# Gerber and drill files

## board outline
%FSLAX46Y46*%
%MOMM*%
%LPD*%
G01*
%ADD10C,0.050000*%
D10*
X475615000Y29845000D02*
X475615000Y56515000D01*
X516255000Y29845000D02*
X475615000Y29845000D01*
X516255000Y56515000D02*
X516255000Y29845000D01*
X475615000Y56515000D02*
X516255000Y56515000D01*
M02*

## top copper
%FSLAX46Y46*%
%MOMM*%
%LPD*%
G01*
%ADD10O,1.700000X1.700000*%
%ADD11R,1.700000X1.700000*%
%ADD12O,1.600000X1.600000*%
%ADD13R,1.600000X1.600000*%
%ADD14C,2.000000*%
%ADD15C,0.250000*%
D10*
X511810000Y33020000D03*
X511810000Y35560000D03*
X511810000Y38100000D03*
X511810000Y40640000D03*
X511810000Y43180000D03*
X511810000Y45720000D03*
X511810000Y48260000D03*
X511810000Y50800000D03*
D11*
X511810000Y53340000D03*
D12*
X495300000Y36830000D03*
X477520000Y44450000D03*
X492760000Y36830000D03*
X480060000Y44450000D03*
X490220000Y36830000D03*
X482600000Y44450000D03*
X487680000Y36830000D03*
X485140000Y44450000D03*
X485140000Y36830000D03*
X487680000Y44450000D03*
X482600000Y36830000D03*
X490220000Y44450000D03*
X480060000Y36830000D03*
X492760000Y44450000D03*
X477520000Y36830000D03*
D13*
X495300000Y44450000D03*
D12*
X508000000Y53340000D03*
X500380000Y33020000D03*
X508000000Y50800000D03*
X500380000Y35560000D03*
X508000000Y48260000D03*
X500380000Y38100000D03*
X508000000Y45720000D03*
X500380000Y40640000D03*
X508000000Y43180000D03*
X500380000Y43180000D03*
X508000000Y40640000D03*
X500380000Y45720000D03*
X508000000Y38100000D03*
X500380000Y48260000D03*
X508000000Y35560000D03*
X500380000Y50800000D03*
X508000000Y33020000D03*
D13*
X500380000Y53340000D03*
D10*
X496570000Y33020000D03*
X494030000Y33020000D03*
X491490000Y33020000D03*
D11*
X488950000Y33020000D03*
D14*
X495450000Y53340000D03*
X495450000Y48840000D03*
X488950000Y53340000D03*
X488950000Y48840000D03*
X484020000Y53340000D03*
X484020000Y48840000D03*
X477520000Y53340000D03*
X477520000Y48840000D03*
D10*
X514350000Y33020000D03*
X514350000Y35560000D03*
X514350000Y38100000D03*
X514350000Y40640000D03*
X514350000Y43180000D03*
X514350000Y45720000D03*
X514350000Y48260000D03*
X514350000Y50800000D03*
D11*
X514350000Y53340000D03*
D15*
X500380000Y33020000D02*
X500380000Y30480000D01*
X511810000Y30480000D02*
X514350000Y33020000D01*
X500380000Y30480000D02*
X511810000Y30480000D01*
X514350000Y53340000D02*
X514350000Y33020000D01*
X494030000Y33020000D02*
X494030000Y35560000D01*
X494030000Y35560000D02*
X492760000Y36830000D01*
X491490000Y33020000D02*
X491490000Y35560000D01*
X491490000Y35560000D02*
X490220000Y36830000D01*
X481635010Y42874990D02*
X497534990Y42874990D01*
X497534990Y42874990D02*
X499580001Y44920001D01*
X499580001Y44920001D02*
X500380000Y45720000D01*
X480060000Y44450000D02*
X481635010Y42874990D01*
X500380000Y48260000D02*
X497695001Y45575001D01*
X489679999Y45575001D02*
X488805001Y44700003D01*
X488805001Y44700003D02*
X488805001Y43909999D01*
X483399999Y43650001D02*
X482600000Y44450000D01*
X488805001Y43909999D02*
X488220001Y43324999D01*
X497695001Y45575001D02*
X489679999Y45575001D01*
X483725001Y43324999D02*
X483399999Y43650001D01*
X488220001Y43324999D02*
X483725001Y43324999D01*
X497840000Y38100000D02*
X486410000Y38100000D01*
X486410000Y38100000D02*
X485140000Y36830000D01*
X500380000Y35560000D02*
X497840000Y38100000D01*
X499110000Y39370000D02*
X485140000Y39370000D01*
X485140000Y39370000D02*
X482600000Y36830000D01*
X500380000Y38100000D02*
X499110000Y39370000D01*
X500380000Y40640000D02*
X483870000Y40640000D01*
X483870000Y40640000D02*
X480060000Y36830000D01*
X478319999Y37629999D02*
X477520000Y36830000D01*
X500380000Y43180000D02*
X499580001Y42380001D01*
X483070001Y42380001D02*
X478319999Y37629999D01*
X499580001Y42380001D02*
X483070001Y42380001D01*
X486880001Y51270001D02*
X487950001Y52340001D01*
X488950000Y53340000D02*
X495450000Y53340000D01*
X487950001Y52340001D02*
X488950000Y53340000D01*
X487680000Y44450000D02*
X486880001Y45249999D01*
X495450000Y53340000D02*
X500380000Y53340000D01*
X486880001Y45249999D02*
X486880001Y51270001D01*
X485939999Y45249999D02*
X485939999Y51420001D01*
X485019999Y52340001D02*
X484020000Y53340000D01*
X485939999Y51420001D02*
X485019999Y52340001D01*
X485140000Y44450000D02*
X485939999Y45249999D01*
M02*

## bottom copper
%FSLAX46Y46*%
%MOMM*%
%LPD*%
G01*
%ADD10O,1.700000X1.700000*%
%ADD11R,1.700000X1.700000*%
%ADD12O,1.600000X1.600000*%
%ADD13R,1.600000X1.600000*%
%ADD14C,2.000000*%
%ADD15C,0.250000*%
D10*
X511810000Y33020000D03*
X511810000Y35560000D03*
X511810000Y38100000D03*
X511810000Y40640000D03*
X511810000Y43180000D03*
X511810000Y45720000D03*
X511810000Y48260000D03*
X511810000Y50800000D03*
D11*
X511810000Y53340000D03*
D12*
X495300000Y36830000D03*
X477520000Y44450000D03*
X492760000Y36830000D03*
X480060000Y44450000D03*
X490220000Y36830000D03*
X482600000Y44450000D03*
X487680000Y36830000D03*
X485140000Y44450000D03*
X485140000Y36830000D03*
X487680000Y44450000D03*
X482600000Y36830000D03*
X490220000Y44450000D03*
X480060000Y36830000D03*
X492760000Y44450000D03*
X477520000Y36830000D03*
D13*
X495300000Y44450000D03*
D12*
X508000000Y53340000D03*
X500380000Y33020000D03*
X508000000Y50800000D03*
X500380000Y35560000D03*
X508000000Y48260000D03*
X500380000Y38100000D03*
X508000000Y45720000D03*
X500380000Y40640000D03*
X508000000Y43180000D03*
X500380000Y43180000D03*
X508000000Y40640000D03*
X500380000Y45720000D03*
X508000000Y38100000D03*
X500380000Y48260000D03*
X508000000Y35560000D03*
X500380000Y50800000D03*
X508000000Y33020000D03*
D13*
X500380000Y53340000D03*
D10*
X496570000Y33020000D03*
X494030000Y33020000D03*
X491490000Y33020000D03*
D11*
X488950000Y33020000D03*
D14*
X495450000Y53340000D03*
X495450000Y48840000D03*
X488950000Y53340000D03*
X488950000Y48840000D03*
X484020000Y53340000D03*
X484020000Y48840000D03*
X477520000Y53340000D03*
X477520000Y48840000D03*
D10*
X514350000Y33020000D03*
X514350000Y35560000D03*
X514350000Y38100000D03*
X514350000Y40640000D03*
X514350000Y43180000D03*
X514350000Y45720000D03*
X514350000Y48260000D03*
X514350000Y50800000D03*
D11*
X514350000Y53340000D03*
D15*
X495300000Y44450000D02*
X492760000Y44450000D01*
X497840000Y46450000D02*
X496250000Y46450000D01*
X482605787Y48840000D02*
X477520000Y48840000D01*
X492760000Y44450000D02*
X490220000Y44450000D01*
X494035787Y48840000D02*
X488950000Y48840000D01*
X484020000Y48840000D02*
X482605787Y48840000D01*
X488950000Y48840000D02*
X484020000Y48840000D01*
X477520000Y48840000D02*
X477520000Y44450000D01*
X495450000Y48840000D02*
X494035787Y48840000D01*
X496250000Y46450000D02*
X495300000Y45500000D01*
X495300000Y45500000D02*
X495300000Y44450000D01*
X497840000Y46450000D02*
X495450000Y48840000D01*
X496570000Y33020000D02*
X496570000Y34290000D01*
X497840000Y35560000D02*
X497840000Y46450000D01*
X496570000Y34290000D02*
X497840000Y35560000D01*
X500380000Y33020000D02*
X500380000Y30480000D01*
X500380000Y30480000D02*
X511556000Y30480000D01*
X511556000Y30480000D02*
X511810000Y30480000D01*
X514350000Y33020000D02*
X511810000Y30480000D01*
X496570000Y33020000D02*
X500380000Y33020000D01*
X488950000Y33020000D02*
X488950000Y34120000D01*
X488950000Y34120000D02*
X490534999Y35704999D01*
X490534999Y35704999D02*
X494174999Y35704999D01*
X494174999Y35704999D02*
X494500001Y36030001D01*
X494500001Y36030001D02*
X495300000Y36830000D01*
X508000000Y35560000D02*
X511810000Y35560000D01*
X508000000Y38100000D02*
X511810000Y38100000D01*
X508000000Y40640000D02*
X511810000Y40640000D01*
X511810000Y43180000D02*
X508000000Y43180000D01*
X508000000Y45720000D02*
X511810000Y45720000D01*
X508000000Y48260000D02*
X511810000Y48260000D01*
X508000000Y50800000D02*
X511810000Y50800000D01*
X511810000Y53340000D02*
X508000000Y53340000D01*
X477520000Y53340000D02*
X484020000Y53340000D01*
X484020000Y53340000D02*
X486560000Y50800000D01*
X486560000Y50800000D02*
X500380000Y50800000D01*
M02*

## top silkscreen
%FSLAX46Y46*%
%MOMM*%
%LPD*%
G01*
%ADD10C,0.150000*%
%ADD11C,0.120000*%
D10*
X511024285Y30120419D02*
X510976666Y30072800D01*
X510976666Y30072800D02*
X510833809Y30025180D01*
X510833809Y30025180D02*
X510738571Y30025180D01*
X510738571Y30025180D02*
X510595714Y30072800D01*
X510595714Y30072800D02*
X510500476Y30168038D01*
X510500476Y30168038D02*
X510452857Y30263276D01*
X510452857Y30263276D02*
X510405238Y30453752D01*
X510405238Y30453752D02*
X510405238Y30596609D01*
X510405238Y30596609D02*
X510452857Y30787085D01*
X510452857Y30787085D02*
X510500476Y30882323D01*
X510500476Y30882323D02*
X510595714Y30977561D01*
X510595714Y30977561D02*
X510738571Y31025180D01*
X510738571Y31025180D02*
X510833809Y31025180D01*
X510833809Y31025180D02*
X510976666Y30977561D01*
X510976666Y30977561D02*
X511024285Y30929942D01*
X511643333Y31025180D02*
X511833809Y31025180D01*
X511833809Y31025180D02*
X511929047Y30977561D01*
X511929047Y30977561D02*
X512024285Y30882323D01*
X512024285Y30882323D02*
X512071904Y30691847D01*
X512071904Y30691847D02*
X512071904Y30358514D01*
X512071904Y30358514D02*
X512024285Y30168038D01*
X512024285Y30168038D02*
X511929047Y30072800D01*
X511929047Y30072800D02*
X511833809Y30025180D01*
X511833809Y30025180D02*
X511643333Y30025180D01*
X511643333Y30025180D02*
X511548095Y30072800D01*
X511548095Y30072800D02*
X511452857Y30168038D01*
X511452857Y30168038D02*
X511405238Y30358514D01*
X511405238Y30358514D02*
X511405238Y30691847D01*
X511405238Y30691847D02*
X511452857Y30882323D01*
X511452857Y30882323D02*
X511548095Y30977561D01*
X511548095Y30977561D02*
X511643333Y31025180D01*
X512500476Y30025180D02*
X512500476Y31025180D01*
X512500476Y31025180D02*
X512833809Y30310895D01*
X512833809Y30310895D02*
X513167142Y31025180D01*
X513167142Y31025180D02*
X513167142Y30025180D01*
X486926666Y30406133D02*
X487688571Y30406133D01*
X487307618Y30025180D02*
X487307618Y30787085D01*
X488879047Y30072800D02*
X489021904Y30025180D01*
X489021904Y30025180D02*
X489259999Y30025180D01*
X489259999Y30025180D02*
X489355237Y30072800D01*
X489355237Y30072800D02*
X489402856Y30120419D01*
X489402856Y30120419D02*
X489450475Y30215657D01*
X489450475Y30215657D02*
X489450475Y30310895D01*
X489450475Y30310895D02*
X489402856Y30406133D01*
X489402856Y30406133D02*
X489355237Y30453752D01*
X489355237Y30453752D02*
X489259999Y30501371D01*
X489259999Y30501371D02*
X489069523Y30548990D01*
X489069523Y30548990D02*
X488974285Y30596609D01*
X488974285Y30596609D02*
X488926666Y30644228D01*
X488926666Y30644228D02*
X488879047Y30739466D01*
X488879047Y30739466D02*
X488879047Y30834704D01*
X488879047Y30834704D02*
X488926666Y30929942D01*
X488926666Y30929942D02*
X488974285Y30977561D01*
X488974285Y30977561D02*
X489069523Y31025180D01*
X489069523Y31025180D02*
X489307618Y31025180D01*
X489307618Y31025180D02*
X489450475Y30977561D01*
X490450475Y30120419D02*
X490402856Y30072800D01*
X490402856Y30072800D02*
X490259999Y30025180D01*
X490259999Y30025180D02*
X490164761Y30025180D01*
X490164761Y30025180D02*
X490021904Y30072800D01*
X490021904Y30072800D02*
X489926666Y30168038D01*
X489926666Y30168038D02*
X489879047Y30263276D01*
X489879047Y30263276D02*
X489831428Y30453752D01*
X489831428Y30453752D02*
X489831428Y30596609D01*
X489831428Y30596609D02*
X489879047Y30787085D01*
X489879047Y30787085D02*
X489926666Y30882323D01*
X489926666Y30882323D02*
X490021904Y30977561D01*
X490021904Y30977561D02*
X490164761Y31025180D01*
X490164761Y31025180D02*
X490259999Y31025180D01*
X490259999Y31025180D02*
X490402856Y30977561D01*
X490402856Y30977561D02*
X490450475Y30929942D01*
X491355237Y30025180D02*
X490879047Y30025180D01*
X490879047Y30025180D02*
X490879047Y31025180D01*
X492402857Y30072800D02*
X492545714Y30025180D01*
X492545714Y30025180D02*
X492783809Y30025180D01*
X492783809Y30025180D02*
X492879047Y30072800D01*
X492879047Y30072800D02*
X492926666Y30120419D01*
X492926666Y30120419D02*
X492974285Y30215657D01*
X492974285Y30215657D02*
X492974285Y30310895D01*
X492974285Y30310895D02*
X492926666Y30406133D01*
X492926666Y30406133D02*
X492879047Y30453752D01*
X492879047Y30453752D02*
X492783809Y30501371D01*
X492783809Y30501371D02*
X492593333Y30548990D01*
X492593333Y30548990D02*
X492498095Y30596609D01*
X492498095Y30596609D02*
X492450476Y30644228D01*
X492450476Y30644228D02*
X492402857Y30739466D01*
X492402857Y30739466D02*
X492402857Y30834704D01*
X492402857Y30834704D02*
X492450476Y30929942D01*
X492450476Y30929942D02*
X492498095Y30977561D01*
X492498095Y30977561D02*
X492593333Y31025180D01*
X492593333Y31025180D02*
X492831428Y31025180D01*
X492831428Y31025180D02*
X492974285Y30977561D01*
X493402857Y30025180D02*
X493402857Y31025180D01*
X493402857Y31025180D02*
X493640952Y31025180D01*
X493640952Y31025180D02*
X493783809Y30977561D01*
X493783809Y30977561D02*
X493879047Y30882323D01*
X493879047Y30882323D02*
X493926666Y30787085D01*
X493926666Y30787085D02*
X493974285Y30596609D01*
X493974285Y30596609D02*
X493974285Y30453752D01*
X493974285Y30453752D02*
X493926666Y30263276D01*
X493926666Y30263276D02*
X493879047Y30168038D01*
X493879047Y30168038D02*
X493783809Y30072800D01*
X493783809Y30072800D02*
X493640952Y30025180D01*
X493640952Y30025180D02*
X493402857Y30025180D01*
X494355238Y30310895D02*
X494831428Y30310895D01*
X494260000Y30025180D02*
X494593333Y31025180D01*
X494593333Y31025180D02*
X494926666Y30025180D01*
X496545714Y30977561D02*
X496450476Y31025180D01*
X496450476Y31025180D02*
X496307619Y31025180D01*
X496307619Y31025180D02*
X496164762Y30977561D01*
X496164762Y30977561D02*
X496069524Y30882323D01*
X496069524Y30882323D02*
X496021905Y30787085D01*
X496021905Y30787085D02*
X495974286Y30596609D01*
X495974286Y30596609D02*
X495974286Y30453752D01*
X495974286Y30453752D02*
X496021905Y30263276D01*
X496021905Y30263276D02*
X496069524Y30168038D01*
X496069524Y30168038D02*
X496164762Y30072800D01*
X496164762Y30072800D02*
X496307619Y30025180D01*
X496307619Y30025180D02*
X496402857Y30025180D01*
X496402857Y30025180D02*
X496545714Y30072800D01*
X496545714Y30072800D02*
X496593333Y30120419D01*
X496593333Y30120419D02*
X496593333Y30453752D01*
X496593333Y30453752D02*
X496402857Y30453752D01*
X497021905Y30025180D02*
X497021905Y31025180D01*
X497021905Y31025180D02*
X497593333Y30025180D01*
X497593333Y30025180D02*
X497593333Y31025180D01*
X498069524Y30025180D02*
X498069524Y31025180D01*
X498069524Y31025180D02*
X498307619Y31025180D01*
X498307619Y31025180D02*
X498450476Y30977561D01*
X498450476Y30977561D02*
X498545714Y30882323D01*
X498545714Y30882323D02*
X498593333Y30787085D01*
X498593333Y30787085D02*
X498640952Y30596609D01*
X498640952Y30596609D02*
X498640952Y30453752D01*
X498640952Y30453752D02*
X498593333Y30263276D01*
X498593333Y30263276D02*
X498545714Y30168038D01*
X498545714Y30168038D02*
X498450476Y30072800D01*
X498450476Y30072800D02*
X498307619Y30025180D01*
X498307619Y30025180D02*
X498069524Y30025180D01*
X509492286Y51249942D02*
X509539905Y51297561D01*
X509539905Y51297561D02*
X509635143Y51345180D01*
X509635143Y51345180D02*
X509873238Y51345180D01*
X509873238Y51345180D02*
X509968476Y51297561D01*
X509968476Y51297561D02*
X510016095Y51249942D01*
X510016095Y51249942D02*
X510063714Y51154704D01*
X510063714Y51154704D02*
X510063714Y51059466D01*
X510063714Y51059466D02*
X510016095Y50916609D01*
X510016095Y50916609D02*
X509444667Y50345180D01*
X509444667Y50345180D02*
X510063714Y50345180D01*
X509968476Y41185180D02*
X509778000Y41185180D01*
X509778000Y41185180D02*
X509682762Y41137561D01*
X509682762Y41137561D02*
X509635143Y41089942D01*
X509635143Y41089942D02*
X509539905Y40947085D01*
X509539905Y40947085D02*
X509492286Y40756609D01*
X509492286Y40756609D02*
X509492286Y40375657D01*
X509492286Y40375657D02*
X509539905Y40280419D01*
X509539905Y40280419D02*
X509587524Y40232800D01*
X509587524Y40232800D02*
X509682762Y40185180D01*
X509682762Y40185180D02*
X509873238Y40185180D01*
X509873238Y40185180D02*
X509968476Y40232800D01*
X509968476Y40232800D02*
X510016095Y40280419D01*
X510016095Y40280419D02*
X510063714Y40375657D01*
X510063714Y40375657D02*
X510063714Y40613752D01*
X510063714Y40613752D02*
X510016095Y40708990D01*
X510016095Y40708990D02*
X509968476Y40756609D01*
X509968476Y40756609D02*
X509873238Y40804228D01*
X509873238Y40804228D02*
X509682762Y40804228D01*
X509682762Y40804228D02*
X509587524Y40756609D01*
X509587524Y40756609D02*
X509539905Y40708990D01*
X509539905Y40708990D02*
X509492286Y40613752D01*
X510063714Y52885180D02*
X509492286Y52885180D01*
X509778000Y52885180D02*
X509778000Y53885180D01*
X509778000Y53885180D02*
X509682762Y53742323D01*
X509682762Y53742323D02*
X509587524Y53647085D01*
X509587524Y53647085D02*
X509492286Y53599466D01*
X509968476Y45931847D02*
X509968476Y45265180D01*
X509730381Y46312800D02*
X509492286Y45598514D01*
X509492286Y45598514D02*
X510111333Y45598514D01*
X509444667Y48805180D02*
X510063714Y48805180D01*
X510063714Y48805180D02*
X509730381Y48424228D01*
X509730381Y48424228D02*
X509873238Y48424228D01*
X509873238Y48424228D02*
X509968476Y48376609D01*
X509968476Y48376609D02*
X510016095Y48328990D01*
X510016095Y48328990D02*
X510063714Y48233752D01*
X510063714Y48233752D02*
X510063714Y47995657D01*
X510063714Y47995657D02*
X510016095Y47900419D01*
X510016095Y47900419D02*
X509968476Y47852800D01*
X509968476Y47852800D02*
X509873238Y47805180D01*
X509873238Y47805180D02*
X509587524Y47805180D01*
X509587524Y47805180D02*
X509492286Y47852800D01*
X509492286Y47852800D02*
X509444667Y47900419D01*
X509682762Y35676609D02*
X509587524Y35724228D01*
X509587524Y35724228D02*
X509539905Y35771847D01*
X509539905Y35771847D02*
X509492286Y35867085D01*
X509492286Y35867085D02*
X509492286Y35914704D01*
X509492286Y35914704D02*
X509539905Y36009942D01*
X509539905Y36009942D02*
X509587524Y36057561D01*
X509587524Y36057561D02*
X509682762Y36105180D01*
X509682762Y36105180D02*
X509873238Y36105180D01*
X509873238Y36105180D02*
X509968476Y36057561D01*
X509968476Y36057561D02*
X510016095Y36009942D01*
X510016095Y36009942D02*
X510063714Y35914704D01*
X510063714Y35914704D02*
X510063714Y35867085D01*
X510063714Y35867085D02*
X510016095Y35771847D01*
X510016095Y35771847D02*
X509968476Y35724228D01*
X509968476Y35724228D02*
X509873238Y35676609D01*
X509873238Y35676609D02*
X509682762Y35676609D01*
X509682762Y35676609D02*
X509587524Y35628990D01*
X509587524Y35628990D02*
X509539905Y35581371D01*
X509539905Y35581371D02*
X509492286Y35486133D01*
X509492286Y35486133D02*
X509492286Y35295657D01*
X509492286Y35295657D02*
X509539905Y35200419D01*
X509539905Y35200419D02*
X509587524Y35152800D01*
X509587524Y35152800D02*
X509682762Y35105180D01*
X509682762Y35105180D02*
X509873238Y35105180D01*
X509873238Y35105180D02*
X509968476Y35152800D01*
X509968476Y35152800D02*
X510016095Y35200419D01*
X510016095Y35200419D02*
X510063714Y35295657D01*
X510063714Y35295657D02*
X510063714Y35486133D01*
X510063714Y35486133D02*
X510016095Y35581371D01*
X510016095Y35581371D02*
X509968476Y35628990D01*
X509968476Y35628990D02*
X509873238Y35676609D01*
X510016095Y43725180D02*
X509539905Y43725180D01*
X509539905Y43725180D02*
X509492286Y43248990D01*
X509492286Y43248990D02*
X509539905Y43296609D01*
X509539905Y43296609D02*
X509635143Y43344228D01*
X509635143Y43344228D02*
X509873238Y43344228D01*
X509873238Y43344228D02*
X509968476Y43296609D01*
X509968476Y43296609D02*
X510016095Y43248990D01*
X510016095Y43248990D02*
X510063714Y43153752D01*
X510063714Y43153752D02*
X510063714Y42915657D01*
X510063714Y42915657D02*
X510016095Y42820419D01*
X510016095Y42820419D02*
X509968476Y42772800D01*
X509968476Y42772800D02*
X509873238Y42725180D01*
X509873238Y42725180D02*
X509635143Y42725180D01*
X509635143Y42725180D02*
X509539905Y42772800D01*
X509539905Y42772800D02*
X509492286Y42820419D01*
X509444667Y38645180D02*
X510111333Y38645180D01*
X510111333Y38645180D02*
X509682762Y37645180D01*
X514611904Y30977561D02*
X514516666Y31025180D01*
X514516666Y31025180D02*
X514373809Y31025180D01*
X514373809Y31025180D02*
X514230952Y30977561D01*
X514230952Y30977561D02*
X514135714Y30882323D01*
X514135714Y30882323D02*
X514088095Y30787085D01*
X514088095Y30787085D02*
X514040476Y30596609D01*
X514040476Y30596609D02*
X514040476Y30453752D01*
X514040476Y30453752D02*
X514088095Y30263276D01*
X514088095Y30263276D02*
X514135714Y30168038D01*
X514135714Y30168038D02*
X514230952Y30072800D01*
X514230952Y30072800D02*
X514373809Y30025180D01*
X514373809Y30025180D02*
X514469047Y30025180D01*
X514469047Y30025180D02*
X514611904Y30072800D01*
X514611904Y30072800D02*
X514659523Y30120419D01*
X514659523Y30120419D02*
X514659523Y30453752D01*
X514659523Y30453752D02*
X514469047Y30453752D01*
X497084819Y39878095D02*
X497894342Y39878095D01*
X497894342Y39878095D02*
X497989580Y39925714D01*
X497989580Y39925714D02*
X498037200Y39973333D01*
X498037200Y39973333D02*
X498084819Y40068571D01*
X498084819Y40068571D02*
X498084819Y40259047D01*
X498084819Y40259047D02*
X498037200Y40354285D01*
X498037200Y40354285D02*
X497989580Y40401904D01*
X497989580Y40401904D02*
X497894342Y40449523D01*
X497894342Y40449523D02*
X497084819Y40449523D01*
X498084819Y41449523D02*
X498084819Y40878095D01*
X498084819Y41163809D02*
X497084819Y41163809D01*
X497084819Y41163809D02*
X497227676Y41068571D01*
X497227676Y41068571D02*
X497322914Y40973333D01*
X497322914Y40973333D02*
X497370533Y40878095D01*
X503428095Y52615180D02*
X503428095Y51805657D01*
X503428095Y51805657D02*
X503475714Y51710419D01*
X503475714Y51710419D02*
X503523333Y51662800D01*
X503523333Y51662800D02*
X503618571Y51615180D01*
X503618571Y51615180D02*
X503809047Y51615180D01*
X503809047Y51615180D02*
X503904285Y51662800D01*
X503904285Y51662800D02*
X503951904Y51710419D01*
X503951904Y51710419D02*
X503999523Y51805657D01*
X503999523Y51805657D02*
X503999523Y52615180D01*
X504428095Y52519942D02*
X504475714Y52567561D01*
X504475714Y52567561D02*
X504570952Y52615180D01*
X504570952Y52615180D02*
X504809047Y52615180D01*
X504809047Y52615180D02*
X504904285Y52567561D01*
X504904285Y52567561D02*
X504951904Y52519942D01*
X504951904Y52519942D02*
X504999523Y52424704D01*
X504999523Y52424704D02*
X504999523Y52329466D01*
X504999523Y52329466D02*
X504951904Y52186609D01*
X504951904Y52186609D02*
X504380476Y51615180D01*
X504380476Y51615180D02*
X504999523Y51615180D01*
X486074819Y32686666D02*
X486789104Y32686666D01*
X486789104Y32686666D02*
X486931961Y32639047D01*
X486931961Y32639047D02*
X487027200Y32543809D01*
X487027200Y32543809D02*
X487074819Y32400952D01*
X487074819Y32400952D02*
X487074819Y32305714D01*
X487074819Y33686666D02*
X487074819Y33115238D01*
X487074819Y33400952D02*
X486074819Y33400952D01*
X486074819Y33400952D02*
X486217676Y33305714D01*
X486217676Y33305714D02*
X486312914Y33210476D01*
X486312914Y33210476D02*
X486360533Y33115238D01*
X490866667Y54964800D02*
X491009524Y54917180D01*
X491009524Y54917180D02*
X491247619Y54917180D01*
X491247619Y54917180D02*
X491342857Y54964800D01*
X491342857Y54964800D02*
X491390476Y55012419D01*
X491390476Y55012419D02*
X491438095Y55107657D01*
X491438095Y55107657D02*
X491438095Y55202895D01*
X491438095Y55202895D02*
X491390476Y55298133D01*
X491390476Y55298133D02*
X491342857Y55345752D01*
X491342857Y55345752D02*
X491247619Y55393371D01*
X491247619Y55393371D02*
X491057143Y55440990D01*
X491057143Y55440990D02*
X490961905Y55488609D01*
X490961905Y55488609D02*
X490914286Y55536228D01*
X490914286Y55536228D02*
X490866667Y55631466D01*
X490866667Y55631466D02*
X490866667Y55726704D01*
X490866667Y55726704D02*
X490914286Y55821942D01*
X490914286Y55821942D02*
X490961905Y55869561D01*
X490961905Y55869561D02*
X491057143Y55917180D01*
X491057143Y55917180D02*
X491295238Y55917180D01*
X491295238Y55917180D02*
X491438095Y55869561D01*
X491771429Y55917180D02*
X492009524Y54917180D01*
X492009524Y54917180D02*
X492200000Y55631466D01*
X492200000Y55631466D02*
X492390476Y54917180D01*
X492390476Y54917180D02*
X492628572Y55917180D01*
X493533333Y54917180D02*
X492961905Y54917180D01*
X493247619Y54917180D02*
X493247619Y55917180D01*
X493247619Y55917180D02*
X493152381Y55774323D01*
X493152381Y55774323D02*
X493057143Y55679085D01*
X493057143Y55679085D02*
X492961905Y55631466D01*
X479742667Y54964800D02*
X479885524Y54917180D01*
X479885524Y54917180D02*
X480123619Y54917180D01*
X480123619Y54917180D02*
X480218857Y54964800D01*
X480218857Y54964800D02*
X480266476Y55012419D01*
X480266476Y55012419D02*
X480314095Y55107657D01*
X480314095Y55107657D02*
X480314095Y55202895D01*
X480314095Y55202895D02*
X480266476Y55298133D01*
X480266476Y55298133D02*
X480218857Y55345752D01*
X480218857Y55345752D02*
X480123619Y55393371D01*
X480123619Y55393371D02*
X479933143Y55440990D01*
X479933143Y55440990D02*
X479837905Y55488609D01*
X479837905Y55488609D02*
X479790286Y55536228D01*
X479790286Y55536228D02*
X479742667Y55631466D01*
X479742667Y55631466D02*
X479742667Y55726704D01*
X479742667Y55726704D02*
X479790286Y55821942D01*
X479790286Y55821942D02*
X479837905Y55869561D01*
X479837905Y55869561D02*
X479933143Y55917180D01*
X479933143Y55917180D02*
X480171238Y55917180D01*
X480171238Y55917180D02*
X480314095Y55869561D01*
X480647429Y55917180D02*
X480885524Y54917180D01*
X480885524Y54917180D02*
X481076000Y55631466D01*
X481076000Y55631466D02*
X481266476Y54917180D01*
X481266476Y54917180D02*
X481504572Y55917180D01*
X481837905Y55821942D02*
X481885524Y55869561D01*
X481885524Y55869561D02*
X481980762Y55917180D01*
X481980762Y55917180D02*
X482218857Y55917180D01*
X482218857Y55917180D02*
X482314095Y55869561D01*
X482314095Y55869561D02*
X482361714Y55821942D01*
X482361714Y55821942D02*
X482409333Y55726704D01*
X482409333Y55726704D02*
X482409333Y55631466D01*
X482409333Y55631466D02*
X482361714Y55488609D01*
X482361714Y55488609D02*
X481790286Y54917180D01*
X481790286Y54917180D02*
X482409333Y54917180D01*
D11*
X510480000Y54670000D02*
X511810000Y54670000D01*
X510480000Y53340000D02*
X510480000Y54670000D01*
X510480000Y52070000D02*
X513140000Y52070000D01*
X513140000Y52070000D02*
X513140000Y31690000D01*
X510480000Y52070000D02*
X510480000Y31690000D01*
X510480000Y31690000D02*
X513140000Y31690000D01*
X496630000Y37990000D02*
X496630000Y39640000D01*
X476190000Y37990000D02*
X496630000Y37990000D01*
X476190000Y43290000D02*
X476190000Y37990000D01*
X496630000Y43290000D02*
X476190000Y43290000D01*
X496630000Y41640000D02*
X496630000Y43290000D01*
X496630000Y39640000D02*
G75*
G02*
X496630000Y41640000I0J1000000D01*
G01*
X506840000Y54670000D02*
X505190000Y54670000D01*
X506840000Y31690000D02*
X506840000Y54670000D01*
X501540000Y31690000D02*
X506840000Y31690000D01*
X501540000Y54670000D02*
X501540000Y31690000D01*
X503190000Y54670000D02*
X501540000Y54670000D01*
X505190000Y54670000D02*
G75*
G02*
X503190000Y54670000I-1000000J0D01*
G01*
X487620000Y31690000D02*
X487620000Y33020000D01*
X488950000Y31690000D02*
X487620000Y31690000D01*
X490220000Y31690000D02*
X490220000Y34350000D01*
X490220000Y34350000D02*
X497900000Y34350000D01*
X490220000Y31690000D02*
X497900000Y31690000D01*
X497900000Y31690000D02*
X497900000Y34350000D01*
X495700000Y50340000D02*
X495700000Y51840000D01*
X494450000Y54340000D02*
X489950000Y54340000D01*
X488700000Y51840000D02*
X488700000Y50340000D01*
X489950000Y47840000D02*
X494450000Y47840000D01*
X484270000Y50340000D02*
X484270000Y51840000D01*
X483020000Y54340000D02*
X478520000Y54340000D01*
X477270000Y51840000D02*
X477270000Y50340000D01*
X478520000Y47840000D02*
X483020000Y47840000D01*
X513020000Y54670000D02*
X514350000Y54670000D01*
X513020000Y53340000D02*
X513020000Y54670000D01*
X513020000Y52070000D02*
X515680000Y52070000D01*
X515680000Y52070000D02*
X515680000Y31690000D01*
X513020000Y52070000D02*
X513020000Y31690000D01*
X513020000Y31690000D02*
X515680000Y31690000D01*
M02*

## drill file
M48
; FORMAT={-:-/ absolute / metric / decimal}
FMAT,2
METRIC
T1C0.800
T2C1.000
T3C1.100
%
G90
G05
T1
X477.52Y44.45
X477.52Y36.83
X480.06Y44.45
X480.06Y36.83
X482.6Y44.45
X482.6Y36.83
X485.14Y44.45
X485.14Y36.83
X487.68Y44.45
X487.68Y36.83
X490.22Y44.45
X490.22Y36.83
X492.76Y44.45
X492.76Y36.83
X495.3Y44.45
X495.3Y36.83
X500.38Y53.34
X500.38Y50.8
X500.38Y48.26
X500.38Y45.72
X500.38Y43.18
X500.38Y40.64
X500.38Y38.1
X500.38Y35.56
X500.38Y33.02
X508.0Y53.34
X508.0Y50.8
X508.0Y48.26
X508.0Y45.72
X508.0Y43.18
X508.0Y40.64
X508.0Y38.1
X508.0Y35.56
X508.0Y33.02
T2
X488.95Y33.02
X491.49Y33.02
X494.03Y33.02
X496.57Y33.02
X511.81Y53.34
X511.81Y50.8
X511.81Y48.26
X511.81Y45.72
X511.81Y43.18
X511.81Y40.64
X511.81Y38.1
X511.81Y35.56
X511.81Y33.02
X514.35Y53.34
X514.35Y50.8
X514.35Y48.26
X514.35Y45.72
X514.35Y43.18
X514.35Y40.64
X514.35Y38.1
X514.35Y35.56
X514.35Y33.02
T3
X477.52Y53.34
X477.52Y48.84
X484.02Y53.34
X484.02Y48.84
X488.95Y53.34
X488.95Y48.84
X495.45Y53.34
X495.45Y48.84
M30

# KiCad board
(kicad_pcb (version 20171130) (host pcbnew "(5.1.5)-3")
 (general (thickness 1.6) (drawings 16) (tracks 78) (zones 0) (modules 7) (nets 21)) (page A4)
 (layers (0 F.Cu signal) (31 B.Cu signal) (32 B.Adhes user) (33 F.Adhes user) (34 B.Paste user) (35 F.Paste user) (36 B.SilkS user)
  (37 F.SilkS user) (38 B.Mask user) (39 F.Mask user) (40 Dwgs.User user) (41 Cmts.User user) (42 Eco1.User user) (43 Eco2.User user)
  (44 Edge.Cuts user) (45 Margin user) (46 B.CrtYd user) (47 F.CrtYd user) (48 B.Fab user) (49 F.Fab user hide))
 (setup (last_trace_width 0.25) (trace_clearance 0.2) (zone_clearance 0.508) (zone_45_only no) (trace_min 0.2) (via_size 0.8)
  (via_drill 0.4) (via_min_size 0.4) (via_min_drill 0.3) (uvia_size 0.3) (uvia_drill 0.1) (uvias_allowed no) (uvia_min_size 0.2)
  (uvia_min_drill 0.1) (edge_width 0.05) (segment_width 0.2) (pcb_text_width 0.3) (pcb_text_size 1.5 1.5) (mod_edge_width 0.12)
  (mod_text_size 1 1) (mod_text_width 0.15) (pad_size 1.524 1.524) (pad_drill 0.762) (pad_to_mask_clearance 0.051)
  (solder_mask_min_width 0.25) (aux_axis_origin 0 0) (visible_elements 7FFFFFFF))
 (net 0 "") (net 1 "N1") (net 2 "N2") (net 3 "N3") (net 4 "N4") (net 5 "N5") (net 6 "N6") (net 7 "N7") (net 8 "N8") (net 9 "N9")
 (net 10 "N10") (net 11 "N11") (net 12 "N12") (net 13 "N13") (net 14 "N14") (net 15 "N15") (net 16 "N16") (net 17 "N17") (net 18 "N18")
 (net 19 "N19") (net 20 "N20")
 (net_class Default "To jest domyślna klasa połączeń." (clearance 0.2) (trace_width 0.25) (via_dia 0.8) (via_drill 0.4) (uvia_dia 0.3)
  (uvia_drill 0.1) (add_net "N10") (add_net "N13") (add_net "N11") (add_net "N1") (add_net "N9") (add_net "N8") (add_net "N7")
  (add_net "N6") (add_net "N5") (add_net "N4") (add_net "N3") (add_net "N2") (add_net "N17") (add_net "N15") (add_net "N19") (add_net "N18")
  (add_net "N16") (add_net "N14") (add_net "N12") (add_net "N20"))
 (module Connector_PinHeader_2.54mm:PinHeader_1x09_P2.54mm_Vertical (layer F.Cu) (at 511.81 -53.34)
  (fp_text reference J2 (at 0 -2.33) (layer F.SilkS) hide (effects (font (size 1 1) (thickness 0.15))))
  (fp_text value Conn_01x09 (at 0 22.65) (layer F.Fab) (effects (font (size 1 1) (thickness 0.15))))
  (fp_line (start -1.33 -1.33) (end 0 -1.33) (layer F.SilkS) (width 0.12))
  (fp_line (start -1.33 0) (end -1.33 -1.33) (layer F.SilkS) (width 0.12))
  (fp_line (start -1.33 1.27) (end 1.33 1.27) (layer F.SilkS) (width 0.12))
  (fp_line (start 1.33 1.27) (end 1.33 21.65) (layer F.SilkS) (width 0.12))
  (fp_line (start -1.33 1.27) (end -1.33 21.65) (layer F.SilkS) (width 0.12))
  (fp_line (start -1.33 21.65) (end 1.33 21.65) (layer F.SilkS) (width 0.12))
  (pad 9 thru_hole oval (at 0 20.32) (size 1.7 1.7) (drill 1) (layers *.Cu *.Mask) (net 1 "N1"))
  (pad 8 thru_hole oval (at 0 17.78) (size 1.7 1.7) (drill 1) (layers *.Cu *.Mask) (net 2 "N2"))
  (pad 7 thru_hole oval (at 0 15.24) (size 1.7 1.7) (drill 1) (layers *.Cu *.Mask) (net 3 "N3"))
  (pad 6 thru_hole oval (at 0 12.7) (size 1.7 1.7) (drill 1) (layers *.Cu *.Mask) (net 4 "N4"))
  (pad 5 thru_hole oval (at 0 10.16) (size 1.7 1.7) (drill 1) (layers *.Cu *.Mask) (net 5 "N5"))
  (pad 4 thru_hole oval (at 0 7.62) (size 1.7 1.7) (drill 1) (layers *.Cu *.Mask) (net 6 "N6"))
  (pad 3 thru_hole oval (at 0 5.08) (size 1.7 1.7) (drill 1) (layers *.Cu *.Mask) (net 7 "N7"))
  (pad 2 thru_hole oval (at 0 2.54) (size 1.7 1.7) (drill 1) (layers *.Cu *.Mask) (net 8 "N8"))
  (pad 1 thru_hole rect (at 0 0) (size 1.7 1.7) (drill 1) (layers *.Cu *.Mask) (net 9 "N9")))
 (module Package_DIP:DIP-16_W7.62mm (layer F.Cu) (at 495.3 -44.45 270)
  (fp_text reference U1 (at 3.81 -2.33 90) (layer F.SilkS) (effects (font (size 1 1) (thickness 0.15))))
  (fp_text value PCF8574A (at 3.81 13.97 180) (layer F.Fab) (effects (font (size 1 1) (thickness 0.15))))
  (fp_line (start 6.46 -1.33) (end 4.81 -1.33) (layer F.SilkS) (width 0.12))
  (fp_line (start 6.46 19.11) (end 6.46 -1.33) (layer F.SilkS) (width 0.12))
  (fp_line (start 1.16 19.11) (end 6.46 19.11) (layer F.SilkS) (width 0.12))
  (fp_line (start 1.16 -1.33) (end 1.16 19.11) (layer F.SilkS) (width 0.12))
  (fp_line (start 2.81 -1.33) (end 1.16 -1.33) (layer F.SilkS) (width 0.12))
  (fp_arc (start 3.81 -1.33) (end 2.81 -1.33) (angle -180) (layer F.SilkS) (width 0.12))
  (pad 16 thru_hole oval (at 7.62 0 270) (size 1.6 1.6) (drill 0.8) (layers *.Cu *.Mask) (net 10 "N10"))
  (pad 8 thru_hole oval (at 0 17.78 270) (size 1.6 1.6) (drill 0.8) (layers *.Cu *.Mask) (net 1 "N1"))
  (pad 15 thru_hole oval (at 7.62 2.54 270) (size 1.6 1.6) (drill 0.8) (layers *.Cu *.Mask) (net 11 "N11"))
  (pad 7 thru_hole oval (at 0 15.24 270) (size 1.6 1.6) (drill 0.8) (layers *.Cu *.Mask) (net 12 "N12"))
  (pad 14 thru_hole oval (at 7.62 5.08 270) (size 1.6 1.6) (drill 0.8) (layers *.Cu *.Mask) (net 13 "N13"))
  (pad 6 thru_hole oval (at 0 12.7 270) (size 1.6 1.6) (drill 0.8) (layers *.Cu *.Mask) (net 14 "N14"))
  (pad 13 thru_hole oval (at 7.62 7.62 270) (size 1.6 1.6) (drill 0.8) (layers *.Cu *.Mask))
  (pad 5 thru_hole oval (at 0 10.16 270) (size 1.6 1.6) (drill 0.8) (layers *.Cu *.Mask) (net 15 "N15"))
  (pad 12 thru_hole oval (at 7.62 10.16 270) (size 1.6 1.6) (drill 0.8) (layers *.Cu *.Mask) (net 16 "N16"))
  (pad 4 thru_hole oval (at 0 7.62 270) (size 1.6 1.6) (drill 0.8) (layers *.Cu *.Mask) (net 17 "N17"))
  (pad 11 thru_hole oval (at 7.62 12.7 270) (size 1.6 1.6) (drill 0.8) (layers *.Cu *.Mask) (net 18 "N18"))
  (pad 3 thru_hole oval (at 0 5.08 270) (size 1.6 1.6) (drill 0.8) (layers *.Cu *.Mask) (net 1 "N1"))
  (pad 10 thru_hole oval (at 7.62 15.24 270) (size 1.6 1.6) (drill 0.8) (layers *.Cu *.Mask) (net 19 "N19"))
  (pad 2 thru_hole oval (at 0 2.54 270) (size 1.6 1.6) (drill 0.8) (layers *.Cu *.Mask) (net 1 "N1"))
  (pad 9 thru_hole oval (at 7.62 17.78 270) (size 1.6 1.6) (drill 0.8) (layers *.Cu *.Mask) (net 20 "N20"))
  (pad 1 thru_hole rect (at 0 0 270) (size 1.6 1.6) (drill 0.8) (layers *.Cu *.Mask) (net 1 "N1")))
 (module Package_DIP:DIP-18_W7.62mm (layer F.Cu) (at 500.38 -53.34)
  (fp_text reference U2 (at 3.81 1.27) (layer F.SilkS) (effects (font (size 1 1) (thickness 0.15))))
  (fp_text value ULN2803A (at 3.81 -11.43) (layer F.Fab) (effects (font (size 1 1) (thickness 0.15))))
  (fp_line (start 6.46 -1.33) (end 4.81 -1.33) (layer F.SilkS) (width 0.12))
  (fp_line (start 6.46 21.65) (end 6.46 -1.33) (layer F.SilkS) (width 0.12))
  (fp_line (start 1.16 21.65) (end 6.46 21.65) (layer F.SilkS) (width 0.12))
  (fp_line (start 1.16 -1.33) (end 1.16 21.65) (layer F.SilkS) (width 0.12))
  (fp_line (start 2.81 -1.33) (end 1.16 -1.33) (layer F.SilkS) (width 0.12))
  (fp_arc (start 3.81 -1.33) (end 2.81 -1.33) (angle -180) (layer F.SilkS) (width 0.12))
  (pad 18 thru_hole oval (at 7.62 0) (size 1.6 1.6) (drill 0.8) (layers *.Cu *.Mask) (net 9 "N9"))
  (pad 9 thru_hole oval (at 0 20.32) (size 1.6 1.6) (drill 0.8) (layers *.Cu *.Mask) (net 1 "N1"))
  (pad 17 thru_hole oval (at 7.62 2.54) (size 1.6 1.6) (drill 0.8) (layers *.Cu *.Mask) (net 8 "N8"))
  (pad 8 thru_hole oval (at 0 17.78) (size 1.6 1.6) (drill 0.8) (layers *.Cu *.Mask) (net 16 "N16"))
  (pad 16 thru_hole oval (at 7.62 5.08) (size 1.6 1.6) (drill 0.8) (layers *.Cu *.Mask) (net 7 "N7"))
  (pad 7 thru_hole oval (at 0 15.24) (size 1.6 1.6) (drill 0.8) (layers *.Cu *.Mask) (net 18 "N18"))
  (pad 15 thru_hole oval (at 7.62 7.62) (size 1.6 1.6) (drill 0.8) (layers *.Cu *.Mask) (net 6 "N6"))
  (pad 6 thru_hole oval (at 0 12.7) (size 1.6 1.6) (drill 0.8) (layers *.Cu *.Mask) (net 19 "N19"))
  (pad 14 thru_hole oval (at 7.62 10.16) (size 1.6 1.6) (drill 0.8) (layers *.Cu *.Mask) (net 5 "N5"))
  (pad 5 thru_hole oval (at 0 10.16) (size 1.6 1.6) (drill 0.8) (layers *.Cu *.Mask) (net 20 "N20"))
  (pad 13 thru_hole oval (at 7.62 12.7) (size 1.6 1.6) (drill 0.8) (layers *.Cu *.Mask) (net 4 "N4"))
  (pad 4 thru_hole oval (at 0 7.62) (size 1.6 1.6) (drill 0.8) (layers *.Cu *.Mask) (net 12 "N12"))
  (pad 12 thru_hole oval (at 7.62 15.24) (size 1.6 1.6) (drill 0.8) (layers *.Cu *.Mask) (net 3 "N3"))
  (pad 3 thru_hole oval (at 0 5.08) (size 1.6 1.6) (drill 0.8) (layers *.Cu *.Mask) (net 14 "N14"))
  (pad 11 thru_hole oval (at 7.62 17.78) (size 1.6 1.6) (drill 0.8) (layers *.Cu *.Mask) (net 2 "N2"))
  (pad 2 thru_hole oval (at 0 2.54) (size 1.6 1.6) (drill 0.8) (layers *.Cu *.Mask) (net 15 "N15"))
  (pad 10 thru_hole oval (at 7.62 20.32) (size 1.6 1.6) (drill 0.8) (layers *.Cu *.Mask))
  (pad 1 thru_hole rect (at 0 0) (size 1.6 1.6) (drill 0.8) (layers *.Cu *.Mask) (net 17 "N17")))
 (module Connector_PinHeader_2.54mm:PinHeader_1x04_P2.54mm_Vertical (layer F.Cu) (at 488.95 -33.02 90)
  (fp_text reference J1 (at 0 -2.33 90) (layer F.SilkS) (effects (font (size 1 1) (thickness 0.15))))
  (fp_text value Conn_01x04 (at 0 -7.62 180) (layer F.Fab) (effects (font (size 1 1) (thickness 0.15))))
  (fp_line (start -1.33 -1.33) (end 0 -1.33) (layer F.SilkS) (width 0.12))
  (fp_line (start -1.33 0) (end -1.33 -1.33) (layer F.SilkS) (width 0.12))
  (fp_line (start -1.33 1.27) (end 1.33 1.27) (layer F.SilkS) (width 0.12))
  (fp_line (start 1.33 1.27) (end 1.33 8.95) (layer F.SilkS) (width 0.12))
  (fp_line (start -1.33 1.27) (end -1.33 8.95) (layer F.SilkS) (width 0.12))
  (fp_line (start -1.33 8.95) (end 1.33 8.95) (layer F.SilkS) (width 0.12))
  (pad 4 thru_hole oval (at 0 7.62 90) (size 1.7 1.7) (drill 1) (layers *.Cu *.Mask) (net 1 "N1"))
  (pad 3 thru_hole oval (at 0 5.08 90) (size 1.7 1.7) (drill 1) (layers *.Cu *.Mask) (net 11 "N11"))
  (pad 2 thru_hole oval (at 0 2.54 90) (size 1.7 1.7) (drill 1) (layers *.Cu *.Mask) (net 13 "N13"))
  (pad 1 thru_hole rect (at 0 0 90) (size 1.7 1.7) (drill 1) (layers *.Cu *.Mask) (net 10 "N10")))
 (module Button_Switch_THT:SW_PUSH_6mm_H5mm (layer F.Cu) (at 488.95 -53.34)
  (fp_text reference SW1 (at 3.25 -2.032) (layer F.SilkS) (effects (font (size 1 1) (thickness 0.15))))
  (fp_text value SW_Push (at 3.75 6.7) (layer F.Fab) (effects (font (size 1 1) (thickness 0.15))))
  (fp_line (start 6.75 3) (end 6.75 1.5) (layer F.SilkS) (width 0.12))
  (fp_line (start 5.5 -1) (end 1 -1) (layer F.SilkS) (width 0.12))
  (fp_line (start -0.25 1.5) (end -0.25 3) (layer F.SilkS) (width 0.12))
  (fp_line (start 1 5.5) (end 5.5 5.5) (layer F.SilkS) (width 0.12))
  (pad 1 thru_hole circle (at 6.5 0 90) (size 2 2) (drill 1.1) (layers *.Cu *.Mask) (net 17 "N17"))
  (pad 2 thru_hole circle (at 6.5 4.5 90) (size 2 2) (drill 1.1) (layers *.Cu *.Mask) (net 1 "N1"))
  (pad 1 thru_hole circle (at 0 0 90) (size 2 2) (drill 1.1) (layers *.Cu *.Mask) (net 17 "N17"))
  (pad 2 thru_hole circle (at 0 4.5 90) (size 2 2) (drill 1.1) (layers *.Cu *.Mask) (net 1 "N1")))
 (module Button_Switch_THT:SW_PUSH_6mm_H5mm (layer F.Cu) (at 477.52 -53.34)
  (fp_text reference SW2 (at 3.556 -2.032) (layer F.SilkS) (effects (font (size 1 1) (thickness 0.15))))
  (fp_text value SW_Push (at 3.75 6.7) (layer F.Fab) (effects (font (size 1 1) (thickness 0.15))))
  (fp_line (start 6.75 3) (end 6.75 1.5) (layer F.SilkS) (width 0.12))
  (fp_line (start 5.5 -1) (end 1 -1) (layer F.SilkS) (width 0.12))
  (fp_line (start -0.25 1.5) (end -0.25 3) (layer F.SilkS) (width 0.12))
  (fp_line (start 1 5.5) (end 5.5 5.5) (layer F.SilkS) (width 0.12))
  (pad 1 thru_hole circle (at 6.5 0 90) (size 2 2) (drill 1.1) (layers *.Cu *.Mask) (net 15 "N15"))
  (pad 2 thru_hole circle (at 6.5 4.5 90) (size 2 2) (drill 1.1) (layers *.Cu *.Mask) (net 1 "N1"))
  (pad 1 thru_hole circle (at 0 0 90) (size 2 2) (drill 1.1) (layers *.Cu *.Mask) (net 15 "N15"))
  (pad 2 thru_hole circle (at 0 4.5 90) (size 2 2) (drill 1.1) (layers *.Cu *.Mask) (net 1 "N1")))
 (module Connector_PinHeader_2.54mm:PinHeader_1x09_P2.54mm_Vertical (layer F.Cu) (at 514.35 -53.34)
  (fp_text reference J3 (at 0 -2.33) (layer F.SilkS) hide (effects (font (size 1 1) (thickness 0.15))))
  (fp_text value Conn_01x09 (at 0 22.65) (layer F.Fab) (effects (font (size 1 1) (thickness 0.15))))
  (fp_line (start -1.33 -1.33) (end 0 -1.33) (layer F.SilkS) (width 0.12))
  (fp_line (start -1.33 0) (end -1.33 -1.33) (layer F.SilkS) (width 0.12))
  (fp_line (start -1.33 1.27) (end 1.33 1.27) (layer F.SilkS) (width 0.12))
  (fp_line (start 1.33 1.27) (end 1.33 21.65) (layer F.SilkS) (width 0.12))
  (fp_line (start -1.33 1.27) (end -1.33 21.65) (layer F.SilkS) (width 0.12))
  (fp_line (start -1.33 21.65) (end 1.33 21.65) (layer F.SilkS) (width 0.12))
  (pad 9 thru_hole oval (at 0 20.32) (size 1.7 1.7) (drill 1) (layers *.Cu *.Mask) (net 1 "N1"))
  (pad 8 thru_hole oval (at 0 17.78) (size 1.7 1.7) (drill 1) (layers *.Cu *.Mask) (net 1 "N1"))
  (pad 7 thru_hole oval (at 0 15.24) (size 1.7 1.7) (drill 1) (layers *.Cu *.Mask) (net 1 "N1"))
  (pad 6 thru_hole oval (at 0 12.7) (size 1.7 1.7) (drill 1) (layers *.Cu *.Mask) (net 1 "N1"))
  (pad 5 thru_hole oval (at 0 10.16) (size 1.7 1.7) (drill 1) (layers *.Cu *.Mask) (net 1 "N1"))
  (pad 4 thru_hole oval (at 0 7.62) (size 1.7 1.7) (drill 1) (layers *.Cu *.Mask) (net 1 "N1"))
  (pad 3 thru_hole oval (at 0 5.08) (size 1.7 1.7) (drill 1) (layers *.Cu *.Mask) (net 1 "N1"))
  (pad 2 thru_hole oval (at 0 2.54) (size 1.7 1.7) (drill 1) (layers *.Cu *.Mask) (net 1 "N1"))
  (pad 1 thru_hole rect (at 0 0) (size 1.7 1.7) (drill 1) (layers *.Cu *.Mask) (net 1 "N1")))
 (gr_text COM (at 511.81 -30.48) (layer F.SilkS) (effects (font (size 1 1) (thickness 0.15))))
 (gr_line (start 475.615 -29.845) (end 475.615 -56.515) (layer Edge.Cuts) (width 0.05))
 (gr_line (start 516.255 -29.845) (end 475.615 -29.845) (layer Edge.Cuts) (width 0.05))
 (gr_line (start 516.255 -56.515) (end 516.255 -29.845) (layer Edge.Cuts) (width 0.05))
 (gr_line (start 475.615 -56.515) (end 516.255 -56.515) (layer Edge.Cuts) (width 0.05))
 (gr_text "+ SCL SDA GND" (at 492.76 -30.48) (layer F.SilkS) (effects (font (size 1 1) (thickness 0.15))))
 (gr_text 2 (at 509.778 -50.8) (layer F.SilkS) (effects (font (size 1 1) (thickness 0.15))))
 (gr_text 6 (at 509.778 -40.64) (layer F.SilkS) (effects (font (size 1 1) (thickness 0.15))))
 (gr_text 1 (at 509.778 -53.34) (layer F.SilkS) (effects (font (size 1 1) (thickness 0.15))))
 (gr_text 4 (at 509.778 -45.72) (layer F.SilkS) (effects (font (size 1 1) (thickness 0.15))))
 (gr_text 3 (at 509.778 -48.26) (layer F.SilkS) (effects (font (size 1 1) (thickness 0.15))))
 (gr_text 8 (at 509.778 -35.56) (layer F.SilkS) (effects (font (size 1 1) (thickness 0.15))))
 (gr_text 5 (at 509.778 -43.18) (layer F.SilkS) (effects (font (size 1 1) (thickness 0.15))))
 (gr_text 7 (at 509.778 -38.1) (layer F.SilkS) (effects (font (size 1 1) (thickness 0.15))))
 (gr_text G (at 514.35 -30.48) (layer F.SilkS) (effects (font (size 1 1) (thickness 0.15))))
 (segment (start 495.3 -44.45) (end 492.76 -44.45) (width 0.25) (layer B.Cu) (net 1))
 (segment (start 497.84 -46.45) (end 496.25 -46.45) (width 0.25) (layer B.Cu) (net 1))
 (segment (start 482.605787 -48.84) (end 477.52 -48.84) (width 0.25) (layer B.Cu) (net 1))
 (segment (start 492.76 -44.45) (end 490.22 -44.45) (width 0.25) (layer B.Cu) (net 1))
 (segment (start 494.035787 -48.84) (end 488.95 -48.84) (width 0.25) (layer B.Cu) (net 1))
 (segment (start 484.02 -48.84) (end 482.605787 -48.84) (width 0.25) (layer B.Cu) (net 1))
 (segment (start 488.95 -48.84) (end 484.02 -48.84) (width 0.25) (layer B.Cu) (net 1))
 (segment (start 477.52 -48.84) (end 477.52 -44.45) (width 0.25) (layer B.Cu) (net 1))
 (segment (start 495.45 -48.84) (end 494.035787 -48.84) (width 0.25) (layer B.Cu) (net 1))
 (segment (start 496.25 -46.45) (end 495.3 -45.5) (width 0.25) (layer B.Cu) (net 1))
 (segment (start 495.3 -45.5) (end 495.3 -44.45) (width 0.25) (layer B.Cu) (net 1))
 (segment (start 497.84 -46.45) (end 495.45 -48.84) (width 0.25) (layer B.Cu) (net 1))
 (segment (start 496.57 -33.02) (end 496.57 -34.29) (width 0.25) (layer B.Cu) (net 1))
 (segment (start 497.84 -35.56) (end 497.84 -46.45) (width 0.25) (layer B.Cu) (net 1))
 (segment (start 496.57 -34.29) (end 497.84 -35.56) (width 0.25) (layer B.Cu) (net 1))
 (segment (start 500.38 -33.02) (end 500.38 -30.48) (width 0.25) (layer B.Cu) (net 1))
 (segment (start 500.38 -33.02) (end 500.38 -30.48) (width 0.25) (layer F.Cu) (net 1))
 (segment (start 500.38 -30.48) (end 511.556 -30.48) (width 0.25) (layer B.Cu) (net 1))
 (segment (start 511.556 -30.48) (end 511.81 -30.48) (width 0.25) (layer B.Cu) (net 1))
 (segment (start 511.81 -30.48) (end 514.35 -33.02) (width 0.25) (layer F.Cu) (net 1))
 (segment (start 500.38 -30.48) (end 511.81 -30.48) (width 0.25) (layer F.Cu) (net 1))
 (segment (start 514.35 -33.02) (end 511.81 -30.48) (width 0.25) (layer B.Cu) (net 1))
 (segment (start 496.57 -33.02) (end 500.38 -33.02) (width 0.25) (layer B.Cu) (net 1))
 (segment (start 514.35 -53.34) (end 514.35 -33.02) (width 0.25) (layer F.Cu) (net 1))
 (segment (start 494.03 -33.02) (end 494.03 -35.56) (width 0.25) (layer F.Cu) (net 11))
 (segment (start 494.03 -35.56) (end 492.76 -36.83) (width 0.25) (layer F.Cu) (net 11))
 (segment (start 491.49 -33.02) (end 491.49 -35.56) (width 0.25) (layer F.Cu) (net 13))
 (segment (start 491.49 -35.56) (end 490.22 -36.83) (width 0.25) (layer F.Cu) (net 13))
 (segment (start 488.95 -33.02) (end 488.95 -34.12) (width 0.25) (layer B.Cu) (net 10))
 (segment (start 488.95 -34.12) (end 490.534999 -35.704999) (width 0.25) (layer B.Cu) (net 10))
 (segment (start 490.534999 -35.704999) (end 494.174999 -35.704999) (width 0.25) (layer B.Cu) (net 10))
 (segment (start 494.174999 -35.704999) (end 494.500001 -36.030001) (width 0.25) (layer B.Cu) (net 10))
 (segment (start 494.500001 -36.030001) (end 495.3 -36.83) (width 0.25) (layer B.Cu) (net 10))
 (segment (start 481.63501 -42.87499) (end 497.53499 -42.87499) (width 0.25) (layer F.Cu) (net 12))
 (segment (start 497.53499 -42.87499) (end 499.580001 -44.920001) (width 0.25) (layer F.Cu) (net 12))
 (segment (start 499.580001 -44.920001) (end 500.38 -45.72) (width 0.25) (layer F.Cu) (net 12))
 (segment (start 480.06 -44.45) (end 481.63501 -42.87499) (width 0.25) (layer F.Cu) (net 12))
 (segment (start 500.38 -48.26) (end 497.695001 -45.575001) (width 0.25) (layer F.Cu) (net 14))
 (segment (start 489.679999 -45.575001) (end 488.805001 -44.700003) (width 0.25) (layer F.Cu) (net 14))
 (segment (start 488.805001 -44.700003) (end 488.805001 -43.909999) (width 0.25) (layer F.Cu) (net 14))
 (segment (start 483.399999 -43.650001) (end 482.6 -44.45) (width 0.25) (layer F.Cu) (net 14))
 (segment (start 488.805001 -43.909999) (end 488.220001 -43.324999) (width 0.25) (layer F.Cu) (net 14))
 (segment (start 497.695001 -45.575001) (end 489.679999 -45.575001) (width 0.25) (layer F.Cu) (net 14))
 (segment (start 483.725001 -43.324999) (end 483.399999 -43.650001) (width 0.25) (layer F.Cu) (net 14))
 (segment (start 488.220001 -43.324999) (end 483.725001 -43.324999) (width 0.25) (layer F.Cu) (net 14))
 (segment (start 497.84 -38.1) (end 486.41 -38.1) (width 0.25) (layer F.Cu) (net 16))
 (segment (start 486.41 -38.1) (end 485.14 -36.83) (width 0.25) (layer F.Cu) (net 16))
 (segment (start 500.38 -35.56) (end 497.84 -38.1) (width 0.25) (layer F.Cu) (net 16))
 (segment (start 499.11 -39.37) (end 485.14 -39.37) (width 0.25) (layer F.Cu) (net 18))
 (segment (start 485.14 -39.37) (end 482.6 -36.83) (width 0.25) (layer F.Cu) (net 18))
 (segment (start 500.38 -38.1) (end 499.11 -39.37) (width 0.25) (layer F.Cu) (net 18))
 (segment (start 500.38 -40.64) (end 483.87 -40.64) (width 0.25) (layer F.Cu) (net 19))
 (segment (start 483.87 -40.64) (end 480.06 -36.83) (width 0.25) (layer F.Cu) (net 19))
 (segment (start 478.319999 -37.629999) (end 477.52 -36.83) (width 0.25) (layer F.Cu) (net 20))
 (segment (start 500.38 -43.18) (end 499.580001 -42.380001) (width 0.25) (layer F.Cu) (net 20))
 (segment (start 483.070001 -42.380001) (end 478.319999 -37.629999) (width 0.25) (layer F.Cu) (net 20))
 (segment (start 499.580001 -42.380001) (end 483.070001 -42.380001) (width 0.25) (layer F.Cu) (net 20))
 (segment (start 508 -35.56) (end 511.81 -35.56) (width 0.25) (layer B.Cu) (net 2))
 (segment (start 508 -38.1) (end 511.81 -38.1) (width 0.25) (layer B.Cu) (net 3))
 (segment (start 508 -40.64) (end 511.81 -40.64) (width 0.25) (layer B.Cu) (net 4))
 (segment (start 511.81 -43.18) (end 508 -43.18) (width 0.25) (layer B.Cu) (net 5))
 (segment (start 508 -45.72) (end 511.81 -45.72) (width 0.25) (layer B.Cu) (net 6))
 (segment (start 508 -48.26) (end 511.81 -48.26) (width 0.25) (layer B.Cu) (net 7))
 (segment (start 508 -50.8) (end 511.81 -50.8) (width 0.25) (layer B.Cu) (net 8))
 (segment (start 511.81 -53.34) (end 508 -53.34) (width 0.25) (layer B.Cu) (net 9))
 (segment (start 486.880001 -51.270001) (end 487.950001 -52.340001) (width 0.25) (layer F.Cu) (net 17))
 (segment (start 488.95 -53.34) (end 495.45 -53.34) (width 0.25) (layer F.Cu) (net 17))
 (segment (start 487.950001 -52.340001) (end 488.95 -53.34) (width 0.25) (layer F.Cu) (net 17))
 (segment (start 487.68 -44.45) (end 486.880001 -45.249999) (width 0.25) (layer F.Cu) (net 17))
 (segment (start 495.45 -53.34) (end 500.38 -53.34) (width 0.25) (layer F.Cu) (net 17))
 (segment (start 486.880001 -45.249999) (end 486.880001 -51.270001) (width 0.25) (layer F.Cu) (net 17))
 (segment (start 485.939999 -45.249999) (end 485.939999 -51.420001) (width 0.25) (layer F.Cu) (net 15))
 (segment (start 485.019999 -52.340001) (end 484.02 -53.34) (width 0.25) (layer F.Cu) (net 15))
 (segment (start 477.52 -53.34) (end 484.02 -53.34) (width 0.25) (layer B.Cu) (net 15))
 (segment (start 484.02 -53.34) (end 486.56 -50.8) (width 0.25) (layer B.Cu) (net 15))
 (segment (start 485.939999 -51.420001) (end 485.019999 -52.340001) (width 0.25) (layer F.Cu) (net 15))
 (segment (start 486.56 -50.8) (end 500.38 -50.8) (width 0.25) (layer B.Cu) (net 15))
 (segment (start 485.14 -44.45) (end 485.939999 -45.249999) (width 0.25) (layer F.Cu) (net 15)))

